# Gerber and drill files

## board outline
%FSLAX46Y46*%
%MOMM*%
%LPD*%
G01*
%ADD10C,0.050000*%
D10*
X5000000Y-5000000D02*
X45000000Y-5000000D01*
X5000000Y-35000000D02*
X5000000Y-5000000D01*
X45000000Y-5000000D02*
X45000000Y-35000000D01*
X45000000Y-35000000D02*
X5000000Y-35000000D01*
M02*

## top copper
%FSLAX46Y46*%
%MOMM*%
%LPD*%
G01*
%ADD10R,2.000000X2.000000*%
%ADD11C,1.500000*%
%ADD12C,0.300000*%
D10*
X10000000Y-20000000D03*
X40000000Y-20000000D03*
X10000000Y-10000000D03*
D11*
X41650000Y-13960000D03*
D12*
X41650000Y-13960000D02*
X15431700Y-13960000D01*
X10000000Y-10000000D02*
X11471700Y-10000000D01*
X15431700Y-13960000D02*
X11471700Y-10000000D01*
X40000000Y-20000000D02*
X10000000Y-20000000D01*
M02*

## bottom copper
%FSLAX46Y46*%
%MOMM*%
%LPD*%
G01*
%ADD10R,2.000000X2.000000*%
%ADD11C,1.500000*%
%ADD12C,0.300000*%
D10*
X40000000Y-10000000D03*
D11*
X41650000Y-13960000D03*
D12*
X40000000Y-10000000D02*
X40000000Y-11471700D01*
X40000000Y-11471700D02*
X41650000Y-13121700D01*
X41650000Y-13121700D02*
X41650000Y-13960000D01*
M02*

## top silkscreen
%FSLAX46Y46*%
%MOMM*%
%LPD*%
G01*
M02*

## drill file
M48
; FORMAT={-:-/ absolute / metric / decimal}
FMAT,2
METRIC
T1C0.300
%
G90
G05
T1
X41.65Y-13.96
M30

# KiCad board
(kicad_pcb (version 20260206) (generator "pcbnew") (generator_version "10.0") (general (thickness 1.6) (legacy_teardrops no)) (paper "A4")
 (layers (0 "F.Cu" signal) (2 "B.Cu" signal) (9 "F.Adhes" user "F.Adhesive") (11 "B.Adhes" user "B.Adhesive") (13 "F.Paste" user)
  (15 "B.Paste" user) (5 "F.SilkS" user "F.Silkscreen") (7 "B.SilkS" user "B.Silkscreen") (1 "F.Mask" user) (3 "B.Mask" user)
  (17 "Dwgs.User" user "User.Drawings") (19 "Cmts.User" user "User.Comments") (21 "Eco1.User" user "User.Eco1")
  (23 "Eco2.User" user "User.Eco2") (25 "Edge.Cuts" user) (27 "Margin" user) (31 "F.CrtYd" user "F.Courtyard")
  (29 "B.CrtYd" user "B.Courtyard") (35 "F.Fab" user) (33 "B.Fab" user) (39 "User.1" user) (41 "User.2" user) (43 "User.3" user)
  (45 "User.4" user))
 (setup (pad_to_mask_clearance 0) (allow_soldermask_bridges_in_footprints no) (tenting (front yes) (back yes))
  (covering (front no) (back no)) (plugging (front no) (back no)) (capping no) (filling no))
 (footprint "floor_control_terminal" (layer "F.Cu") (at 10 20)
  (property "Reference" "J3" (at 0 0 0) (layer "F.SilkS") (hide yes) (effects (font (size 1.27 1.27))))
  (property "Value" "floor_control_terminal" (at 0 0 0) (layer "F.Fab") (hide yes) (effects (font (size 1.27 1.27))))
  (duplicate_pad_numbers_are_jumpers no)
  (pad "1" smd rect (at 0 0) (size 2 2) (layers "F.Cu" "F.Mask" "F.Paste") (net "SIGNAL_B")))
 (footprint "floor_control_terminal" (layer "F.Cu") (at 40 20)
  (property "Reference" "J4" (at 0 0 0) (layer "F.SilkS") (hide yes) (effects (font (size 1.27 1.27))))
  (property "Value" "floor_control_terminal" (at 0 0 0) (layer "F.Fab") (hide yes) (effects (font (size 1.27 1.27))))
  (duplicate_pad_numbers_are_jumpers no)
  (pad "1" smd rect (at 0 0) (size 2 2) (layers "F.Cu" "F.Mask" "F.Paste") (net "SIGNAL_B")))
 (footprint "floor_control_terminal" (layer "F.Cu") (at 10 10)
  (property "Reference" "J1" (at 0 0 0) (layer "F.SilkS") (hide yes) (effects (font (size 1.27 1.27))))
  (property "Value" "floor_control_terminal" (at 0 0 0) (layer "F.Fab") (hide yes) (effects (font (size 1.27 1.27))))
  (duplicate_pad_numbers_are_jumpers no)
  (pad "1" smd rect (at 0 0) (size 2 2) (layers "F.Cu" "F.Mask" "F.Paste") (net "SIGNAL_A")))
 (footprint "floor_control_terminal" (layer "B.Cu") (at 40 10)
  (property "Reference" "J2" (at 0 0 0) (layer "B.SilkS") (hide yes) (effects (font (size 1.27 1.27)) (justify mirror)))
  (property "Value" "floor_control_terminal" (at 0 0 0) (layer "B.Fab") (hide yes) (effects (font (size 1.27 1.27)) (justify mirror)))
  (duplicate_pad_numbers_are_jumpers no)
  (pad "1" smd rect (at 0 0) (size 2 2) (layers "B.Cu" "B.Mask" "B.Paste") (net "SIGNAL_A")))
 (gr_line (start 5 5) (end 45 5) (stroke (width 0.05) (type default)) (layer "Edge.Cuts"))
 (gr_line (start 5 35) (end 5 5) (stroke (width 0.05) (type default)) (layer "Edge.Cuts"))
 (gr_line (start 45 5) (end 45 35) (stroke (width 0.05) (type default)) (layer "Edge.Cuts"))
 (gr_line (start 45 35) (end 5 35) (stroke (width 0.05) (type default)) (layer "Edge.Cuts"))
 (segment (start 41.65 13.96) (end 15.4317 13.96) (width 0.3) (layer "F.Cu") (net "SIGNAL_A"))
 (segment (start 10 10) (end 11.4717 10) (width 0.3) (layer "F.Cu") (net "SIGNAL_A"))
 (segment (start 15.4317 13.96) (end 11.4717 10) (width 0.3) (layer "F.Cu") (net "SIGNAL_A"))
 (via (at 41.65 13.96) (size 1.5) (drill 0.3) (layers "F.Cu" "B.Cu") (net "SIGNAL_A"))
 (segment (start 40 10) (end 40 11.4717) (width 0.3) (layer "B.Cu") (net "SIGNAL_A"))
 (segment (start 40 11.4717) (end 41.65 13.1217) (width 0.3) (layer "B.Cu") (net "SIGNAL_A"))
 (segment (start 41.65 13.1217) (end 41.65 13.96) (width 0.3) (layer "B.Cu") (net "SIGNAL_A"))
 (segment (start 40 20) (end 10 20) (width 0.3) (layer "F.Cu") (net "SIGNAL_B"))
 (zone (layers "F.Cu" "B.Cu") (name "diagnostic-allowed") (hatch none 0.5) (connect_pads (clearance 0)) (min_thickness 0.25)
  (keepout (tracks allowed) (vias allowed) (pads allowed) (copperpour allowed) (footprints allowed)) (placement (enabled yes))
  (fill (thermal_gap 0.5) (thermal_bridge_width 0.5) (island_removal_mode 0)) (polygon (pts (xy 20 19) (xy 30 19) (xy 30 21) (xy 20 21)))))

